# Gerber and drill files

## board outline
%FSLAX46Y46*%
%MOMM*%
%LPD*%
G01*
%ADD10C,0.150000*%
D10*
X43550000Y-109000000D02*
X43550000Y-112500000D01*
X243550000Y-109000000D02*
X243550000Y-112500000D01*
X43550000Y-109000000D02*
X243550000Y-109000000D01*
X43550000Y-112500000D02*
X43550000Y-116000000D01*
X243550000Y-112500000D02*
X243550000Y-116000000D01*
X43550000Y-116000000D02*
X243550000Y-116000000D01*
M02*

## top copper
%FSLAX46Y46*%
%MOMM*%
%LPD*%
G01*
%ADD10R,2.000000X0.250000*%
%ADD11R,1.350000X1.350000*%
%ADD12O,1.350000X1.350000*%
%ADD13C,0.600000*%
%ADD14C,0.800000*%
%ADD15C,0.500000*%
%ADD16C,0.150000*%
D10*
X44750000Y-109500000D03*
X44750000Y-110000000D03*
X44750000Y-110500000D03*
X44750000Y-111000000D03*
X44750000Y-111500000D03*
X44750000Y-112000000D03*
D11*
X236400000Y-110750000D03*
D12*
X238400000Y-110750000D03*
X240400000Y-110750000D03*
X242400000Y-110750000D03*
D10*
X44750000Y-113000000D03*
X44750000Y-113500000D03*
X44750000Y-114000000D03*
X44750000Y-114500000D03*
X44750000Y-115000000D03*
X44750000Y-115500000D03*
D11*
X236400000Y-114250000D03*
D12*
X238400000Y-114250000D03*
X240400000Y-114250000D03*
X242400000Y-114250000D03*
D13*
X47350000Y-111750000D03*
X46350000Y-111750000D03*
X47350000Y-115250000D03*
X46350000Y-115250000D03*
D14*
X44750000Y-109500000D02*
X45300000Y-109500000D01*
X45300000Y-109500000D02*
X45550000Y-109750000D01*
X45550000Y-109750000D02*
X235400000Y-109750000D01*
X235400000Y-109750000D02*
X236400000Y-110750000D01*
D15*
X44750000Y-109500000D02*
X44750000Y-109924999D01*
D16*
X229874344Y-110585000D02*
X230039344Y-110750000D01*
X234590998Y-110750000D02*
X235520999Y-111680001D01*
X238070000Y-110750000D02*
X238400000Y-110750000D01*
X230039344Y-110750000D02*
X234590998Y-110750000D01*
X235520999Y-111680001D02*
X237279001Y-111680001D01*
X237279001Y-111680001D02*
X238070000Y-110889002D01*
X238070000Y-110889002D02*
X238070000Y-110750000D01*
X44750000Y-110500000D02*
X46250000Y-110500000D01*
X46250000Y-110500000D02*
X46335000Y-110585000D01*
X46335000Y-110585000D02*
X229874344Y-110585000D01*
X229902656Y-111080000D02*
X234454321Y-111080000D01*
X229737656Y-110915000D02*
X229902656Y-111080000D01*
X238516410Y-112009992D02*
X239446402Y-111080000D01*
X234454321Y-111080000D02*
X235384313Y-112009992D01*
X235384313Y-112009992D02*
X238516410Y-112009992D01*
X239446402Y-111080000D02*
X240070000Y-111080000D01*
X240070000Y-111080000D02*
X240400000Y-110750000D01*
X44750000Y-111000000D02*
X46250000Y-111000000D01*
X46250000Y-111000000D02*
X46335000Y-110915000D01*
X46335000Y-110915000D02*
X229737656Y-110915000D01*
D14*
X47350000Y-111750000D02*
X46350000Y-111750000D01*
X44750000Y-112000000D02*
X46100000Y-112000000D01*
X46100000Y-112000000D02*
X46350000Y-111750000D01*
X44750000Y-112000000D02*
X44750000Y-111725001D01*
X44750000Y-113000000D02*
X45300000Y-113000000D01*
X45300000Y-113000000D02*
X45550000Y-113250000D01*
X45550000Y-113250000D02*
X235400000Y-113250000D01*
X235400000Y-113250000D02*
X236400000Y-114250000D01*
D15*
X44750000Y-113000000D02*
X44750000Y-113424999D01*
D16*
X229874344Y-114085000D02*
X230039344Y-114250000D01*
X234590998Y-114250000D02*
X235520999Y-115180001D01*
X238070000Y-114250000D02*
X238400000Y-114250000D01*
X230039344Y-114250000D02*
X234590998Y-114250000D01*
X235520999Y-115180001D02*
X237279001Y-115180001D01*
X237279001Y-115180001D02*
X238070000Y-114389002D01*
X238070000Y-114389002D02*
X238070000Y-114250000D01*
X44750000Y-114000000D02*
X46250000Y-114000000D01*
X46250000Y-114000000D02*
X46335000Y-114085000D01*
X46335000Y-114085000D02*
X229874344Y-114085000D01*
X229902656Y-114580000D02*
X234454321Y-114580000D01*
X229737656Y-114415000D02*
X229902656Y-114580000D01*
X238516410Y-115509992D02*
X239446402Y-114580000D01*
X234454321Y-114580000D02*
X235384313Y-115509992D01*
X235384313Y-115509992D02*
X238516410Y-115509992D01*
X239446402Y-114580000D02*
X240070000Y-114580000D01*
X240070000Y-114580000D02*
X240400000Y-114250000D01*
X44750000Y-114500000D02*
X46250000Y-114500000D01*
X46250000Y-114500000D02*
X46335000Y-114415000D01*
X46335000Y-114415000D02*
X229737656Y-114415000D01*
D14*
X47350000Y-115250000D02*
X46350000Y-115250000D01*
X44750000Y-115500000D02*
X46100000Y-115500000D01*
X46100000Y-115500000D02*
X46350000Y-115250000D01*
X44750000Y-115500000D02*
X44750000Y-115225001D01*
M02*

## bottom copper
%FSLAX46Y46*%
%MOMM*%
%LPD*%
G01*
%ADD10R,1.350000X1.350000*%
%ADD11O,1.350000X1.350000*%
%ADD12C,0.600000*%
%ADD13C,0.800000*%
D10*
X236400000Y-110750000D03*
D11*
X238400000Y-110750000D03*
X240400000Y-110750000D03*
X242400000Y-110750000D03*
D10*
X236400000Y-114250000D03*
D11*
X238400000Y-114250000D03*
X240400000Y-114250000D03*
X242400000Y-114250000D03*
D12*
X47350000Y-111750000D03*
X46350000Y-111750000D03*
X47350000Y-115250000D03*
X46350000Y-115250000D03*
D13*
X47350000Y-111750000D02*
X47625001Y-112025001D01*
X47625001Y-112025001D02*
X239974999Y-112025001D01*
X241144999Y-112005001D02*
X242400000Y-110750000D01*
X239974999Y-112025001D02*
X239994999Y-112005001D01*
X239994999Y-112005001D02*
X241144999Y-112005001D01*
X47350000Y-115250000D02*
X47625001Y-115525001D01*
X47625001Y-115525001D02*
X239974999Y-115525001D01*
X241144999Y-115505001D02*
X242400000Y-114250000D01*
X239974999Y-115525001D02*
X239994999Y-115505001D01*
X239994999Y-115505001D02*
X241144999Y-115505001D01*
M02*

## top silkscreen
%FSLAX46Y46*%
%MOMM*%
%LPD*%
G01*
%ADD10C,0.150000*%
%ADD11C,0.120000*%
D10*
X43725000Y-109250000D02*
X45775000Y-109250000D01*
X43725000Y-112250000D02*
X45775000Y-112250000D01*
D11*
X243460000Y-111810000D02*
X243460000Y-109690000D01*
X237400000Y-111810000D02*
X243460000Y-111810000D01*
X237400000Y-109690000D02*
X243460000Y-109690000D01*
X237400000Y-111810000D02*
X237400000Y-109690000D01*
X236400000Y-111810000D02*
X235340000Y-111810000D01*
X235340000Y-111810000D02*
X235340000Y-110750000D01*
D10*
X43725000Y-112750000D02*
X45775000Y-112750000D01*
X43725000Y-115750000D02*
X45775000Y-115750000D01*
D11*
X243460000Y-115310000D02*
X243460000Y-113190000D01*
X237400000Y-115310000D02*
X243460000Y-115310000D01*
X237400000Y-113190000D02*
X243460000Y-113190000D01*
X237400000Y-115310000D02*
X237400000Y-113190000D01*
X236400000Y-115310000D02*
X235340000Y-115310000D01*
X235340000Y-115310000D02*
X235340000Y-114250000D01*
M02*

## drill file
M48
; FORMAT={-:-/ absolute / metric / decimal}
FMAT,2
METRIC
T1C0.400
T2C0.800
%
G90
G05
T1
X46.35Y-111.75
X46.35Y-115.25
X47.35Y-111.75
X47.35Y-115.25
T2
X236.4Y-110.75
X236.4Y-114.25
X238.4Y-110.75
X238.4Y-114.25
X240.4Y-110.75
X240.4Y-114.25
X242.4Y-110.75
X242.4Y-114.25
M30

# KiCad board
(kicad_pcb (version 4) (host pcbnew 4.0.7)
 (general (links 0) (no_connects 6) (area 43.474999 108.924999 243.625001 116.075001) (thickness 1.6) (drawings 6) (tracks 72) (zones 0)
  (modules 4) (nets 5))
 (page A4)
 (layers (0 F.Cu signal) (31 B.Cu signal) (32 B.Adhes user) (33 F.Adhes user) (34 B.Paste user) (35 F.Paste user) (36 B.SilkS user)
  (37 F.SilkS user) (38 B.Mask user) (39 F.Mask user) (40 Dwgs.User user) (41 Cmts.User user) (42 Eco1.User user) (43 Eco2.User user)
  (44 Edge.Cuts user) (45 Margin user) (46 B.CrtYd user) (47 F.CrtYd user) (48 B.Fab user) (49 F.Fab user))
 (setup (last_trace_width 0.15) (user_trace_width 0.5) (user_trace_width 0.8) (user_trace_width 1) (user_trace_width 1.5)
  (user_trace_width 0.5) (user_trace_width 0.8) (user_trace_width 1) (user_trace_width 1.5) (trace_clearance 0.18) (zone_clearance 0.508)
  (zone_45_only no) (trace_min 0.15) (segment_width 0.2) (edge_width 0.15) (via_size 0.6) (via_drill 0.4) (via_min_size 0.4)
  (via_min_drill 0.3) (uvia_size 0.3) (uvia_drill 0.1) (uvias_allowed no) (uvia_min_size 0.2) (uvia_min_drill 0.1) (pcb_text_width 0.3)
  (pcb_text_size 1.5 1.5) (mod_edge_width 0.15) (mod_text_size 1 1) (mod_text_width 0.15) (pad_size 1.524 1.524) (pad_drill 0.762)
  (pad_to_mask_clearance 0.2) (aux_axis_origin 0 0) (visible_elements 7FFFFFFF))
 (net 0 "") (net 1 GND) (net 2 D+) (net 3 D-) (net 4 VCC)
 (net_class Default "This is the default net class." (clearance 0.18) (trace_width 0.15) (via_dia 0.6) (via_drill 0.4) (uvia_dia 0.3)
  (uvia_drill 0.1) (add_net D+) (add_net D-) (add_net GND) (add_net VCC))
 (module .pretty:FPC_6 (layer F.Cu) (at 44.75 110.75 270)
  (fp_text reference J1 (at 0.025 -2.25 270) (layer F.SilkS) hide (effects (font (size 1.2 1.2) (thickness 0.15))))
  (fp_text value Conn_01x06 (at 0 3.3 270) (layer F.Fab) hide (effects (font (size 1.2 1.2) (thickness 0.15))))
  (fp_line (start -1.5 1.025) (end -1.5 -1.025) (layer F.SilkS) (width 0.15))
  (fp_line (start 1.5 1.025) (end 1.5 -1.025) (layer F.SilkS) (width 0.15))
  (pad 1 smd rect (at -1.25 0 270) (size 0.25 2) (layers F.Cu F.Paste F.Mask) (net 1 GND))
  (pad 2 smd rect (at -0.75 0 270) (size 0.25 2) (layers F.Cu F.Paste F.Mask) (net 1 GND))
  (pad 3 smd rect (at -0.25 0 270) (size 0.25 2) (layers F.Cu F.Paste F.Mask) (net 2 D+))
  (pad 4 smd rect (at 0.25 0 270) (size 0.25 2) (layers F.Cu F.Paste F.Mask) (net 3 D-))
  (pad 5 smd rect (at 0.75 0 270) (size 0.25 2) (layers F.Cu F.Paste F.Mask) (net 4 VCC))
  (pad 6 smd rect (at 1.25 0 270) (size 0.25 2) (layers F.Cu F.Paste F.Mask) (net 4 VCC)))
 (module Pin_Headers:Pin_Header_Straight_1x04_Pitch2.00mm (layer F.Cu) (at 236.4 110.75 90)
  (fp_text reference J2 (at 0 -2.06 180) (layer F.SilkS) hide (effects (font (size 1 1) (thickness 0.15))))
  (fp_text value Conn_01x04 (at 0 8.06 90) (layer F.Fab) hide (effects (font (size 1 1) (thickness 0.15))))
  (fp_line (start -1.06 7.06) (end 1.06 7.06) (layer F.SilkS) (width 0.12))
  (fp_line (start -1.06 1) (end -1.06 7.06) (layer F.SilkS) (width 0.12))
  (fp_line (start 1.06 1) (end 1.06 7.06) (layer F.SilkS) (width 0.12))
  (fp_line (start -1.06 1) (end 1.06 1) (layer F.SilkS) (width 0.12))
  (fp_line (start -1.06 0) (end -1.06 -1.06) (layer F.SilkS) (width 0.12))
  (fp_line (start -1.06 -1.06) (end 0 -1.06) (layer F.SilkS) (width 0.12))
  (pad 1 thru_hole rect (at 0 0 90) (size 1.35 1.35) (drill 0.8) (layers *.Cu *.Mask) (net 1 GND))
  (pad 2 thru_hole oval (at 0 2 90) (size 1.35 1.35) (drill 0.8) (layers *.Cu *.Mask) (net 2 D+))
  (pad 3 thru_hole oval (at 0 4 90) (size 1.35 1.35) (drill 0.8) (layers *.Cu *.Mask) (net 3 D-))
  (pad 4 thru_hole oval (at 0 6 90) (size 1.35 1.35) (drill 0.8) (layers *.Cu *.Mask) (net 4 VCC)))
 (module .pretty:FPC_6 (layer F.Cu) (at 44.75 114.25 270)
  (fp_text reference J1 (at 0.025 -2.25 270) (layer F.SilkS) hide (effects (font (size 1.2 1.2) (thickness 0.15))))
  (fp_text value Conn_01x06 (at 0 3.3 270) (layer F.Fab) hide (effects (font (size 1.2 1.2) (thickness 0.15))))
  (fp_line (start -1.5 1.025) (end -1.5 -1.025) (layer F.SilkS) (width 0.15))
  (fp_line (start 1.5 1.025) (end 1.5 -1.025) (layer F.SilkS) (width 0.15))
  (pad 1 smd rect (at -1.25 0 270) (size 0.25 2) (layers F.Cu F.Paste F.Mask) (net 1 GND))
  (pad 2 smd rect (at -0.75 0 270) (size 0.25 2) (layers F.Cu F.Paste F.Mask) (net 1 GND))
  (pad 3 smd rect (at -0.25 0 270) (size 0.25 2) (layers F.Cu F.Paste F.Mask) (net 2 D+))
  (pad 4 smd rect (at 0.25 0 270) (size 0.25 2) (layers F.Cu F.Paste F.Mask) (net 3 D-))
  (pad 5 smd rect (at 0.75 0 270) (size 0.25 2) (layers F.Cu F.Paste F.Mask) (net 4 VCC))
  (pad 6 smd rect (at 1.25 0 270) (size 0.25 2) (layers F.Cu F.Paste F.Mask) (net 4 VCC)))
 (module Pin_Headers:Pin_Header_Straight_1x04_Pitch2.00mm (layer F.Cu) (at 236.4 114.25 90)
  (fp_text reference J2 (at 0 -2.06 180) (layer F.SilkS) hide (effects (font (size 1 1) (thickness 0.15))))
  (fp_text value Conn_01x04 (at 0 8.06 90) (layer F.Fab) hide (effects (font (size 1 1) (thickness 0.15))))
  (fp_line (start -1.06 7.06) (end 1.06 7.06) (layer F.SilkS) (width 0.12))
  (fp_line (start -1.06 1) (end -1.06 7.06) (layer F.SilkS) (width 0.12))
  (fp_line (start 1.06 1) (end 1.06 7.06) (layer F.SilkS) (width 0.12))
  (fp_line (start -1.06 1) (end 1.06 1) (layer F.SilkS) (width 0.12))
  (fp_line (start -1.06 0) (end -1.06 -1.06) (layer F.SilkS) (width 0.12))
  (fp_line (start -1.06 -1.06) (end 0 -1.06) (layer F.SilkS) (width 0.12))
  (pad 1 thru_hole rect (at 0 0 90) (size 1.35 1.35) (drill 0.8) (layers *.Cu *.Mask) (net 1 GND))
  (pad 2 thru_hole oval (at 0 2 90) (size 1.35 1.35) (drill 0.8) (layers *.Cu *.Mask) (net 2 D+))
  (pad 3 thru_hole oval (at 0 4 90) (size 1.35 1.35) (drill 0.8) (layers *.Cu *.Mask) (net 3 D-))
  (pad 4 thru_hole oval (at 0 6 90) (size 1.35 1.35) (drill 0.8) (layers *.Cu *.Mask) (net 4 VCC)))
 (gr_line (start 43.55 109) (end 43.55 112.5) (layer Edge.Cuts) (width 0.15))
 (gr_line (start 243.55 109) (end 243.55 112.5) (layer Edge.Cuts) (width 0.15))
 (gr_line (start 43.55 109) (end 243.55 109) (layer Edge.Cuts) (width 0.15))
 (gr_line (start 43.55 112.5) (end 43.55 116) (layer Edge.Cuts) (width 0.15))
 (gr_line (start 243.55 112.5) (end 243.55 116) (layer Edge.Cuts) (width 0.15))
 (gr_line (start 43.55 116) (end 243.55 116) (layer Edge.Cuts) (width 0.15))
 (segment (start 44.75 109.5) (end 45.3 109.5) (width 0.8) (layer F.Cu) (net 1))
 (segment (start 45.3 109.5) (end 45.55 109.75) (width 0.8) (layer F.Cu) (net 1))
 (segment (start 45.55 109.75) (end 235.4 109.75) (width 0.8) (layer F.Cu) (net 1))
 (segment (start 235.4 109.75) (end 236.4 110.75) (width 0.8) (layer F.Cu) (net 1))
 (segment (start 44.75 109.5) (end 44.75 109.924999) (width 0.5) (layer F.Cu) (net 1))
 (segment (start 229.874344 110.585) (end 230.039344 110.75) (width 0.15) (layer F.Cu) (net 2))
 (segment (start 234.590998 110.75) (end 235.520999 111.680001) (width 0.15) (layer F.Cu) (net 2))
 (segment (start 238.07 110.75) (end 238.4 110.75) (width 0.15) (layer F.Cu) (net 2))
 (segment (start 230.039344 110.75) (end 234.590998 110.75) (width 0.15) (layer F.Cu) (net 2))
 (segment (start 235.520999 111.680001) (end 237.279001 111.680001) (width 0.15) (layer F.Cu) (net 2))
 (segment (start 237.279001 111.680001) (end 238.07 110.889002) (width 0.15) (layer F.Cu) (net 2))
 (segment (start 238.07 110.889002) (end 238.07 110.75) (width 0.15) (layer F.Cu) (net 2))
 (segment (start 44.75 110.5) (end 46.25 110.5) (width 0.15) (layer F.Cu) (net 2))
 (segment (start 46.25 110.5) (end 46.335 110.585) (width 0.15) (layer F.Cu) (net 2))
 (segment (start 46.335 110.585) (end 229.874344 110.585) (width 0.15) (layer F.Cu) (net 2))
 (segment (start 229.902656 111.08) (end 234.454321 111.08) (width 0.15) (layer F.Cu) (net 3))
 (segment (start 229.737656 110.915) (end 229.902656 111.08) (width 0.15) (layer F.Cu) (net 3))
 (segment (start 238.51641 112.009992) (end 239.446402 111.08) (width 0.15) (layer F.Cu) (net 3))
 (segment (start 234.454321 111.08) (end 235.384313 112.009992) (width 0.15) (layer F.Cu) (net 3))
 (segment (start 235.384313 112.009992) (end 238.51641 112.009992) (width 0.15) (layer F.Cu) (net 3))
 (segment (start 239.446402 111.08) (end 240.07 111.08) (width 0.15) (layer F.Cu) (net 3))
 (segment (start 240.07 111.08) (end 240.4 110.75) (width 0.15) (layer F.Cu) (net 3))
 (segment (start 44.75 111) (end 46.25 111) (width 0.15) (layer F.Cu) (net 3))
 (segment (start 46.25 111) (end 46.335 110.915) (width 0.15) (layer F.Cu) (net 3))
 (segment (start 46.335 110.915) (end 229.737656 110.915) (width 0.15) (layer F.Cu) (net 3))
 (segment (start 47.35 111.75) (end 47.625001 112.025001) (width 0.8) (layer B.Cu) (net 4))
 (segment (start 47.625001 112.025001) (end 239.974999 112.025001) (width 0.8) (layer B.Cu) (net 4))
 (segment (start 241.144999 112.005001) (end 242.4 110.75) (width 0.8) (layer B.Cu) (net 4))
 (segment (start 239.974999 112.025001) (end 239.994999 112.005001) (width 0.8) (layer B.Cu) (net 4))
 (segment (start 239.994999 112.005001) (end 241.144999 112.005001) (width 0.8) (layer B.Cu) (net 4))
 (segment (start 47.35 111.75) (end 46.35 111.75) (width 0.8) (layer F.Cu) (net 4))
 (via (at 47.35 111.75) (size 0.6) (drill 0.4) (layers F.Cu B.Cu) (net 4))
 (segment (start 44.75 112) (end 46.1 112) (width 0.8) (layer F.Cu) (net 4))
 (segment (start 46.1 112) (end 46.35 111.75) (width 0.8) (layer F.Cu) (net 4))
 (via (at 46.35 111.75) (size 0.6) (drill 0.4) (layers F.Cu B.Cu) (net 4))
 (segment (start 44.75 112) (end 44.75 111.725001) (width 0.8) (layer F.Cu) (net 4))
 (segment (start 44.75 113) (end 45.3 113) (width 0.8) (layer F.Cu) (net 1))
 (segment (start 45.3 113) (end 45.55 113.25) (width 0.8) (layer F.Cu) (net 1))
 (segment (start 45.55 113.25) (end 235.4 113.25) (width 0.8) (layer F.Cu) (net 1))
 (segment (start 235.4 113.25) (end 236.4 114.25) (width 0.8) (layer F.Cu) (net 1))
 (segment (start 44.75 113) (end 44.75 113.424999) (width 0.5) (layer F.Cu) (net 1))
 (segment (start 229.874344 114.085) (end 230.039344 114.25) (width 0.15) (layer F.Cu) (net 2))
 (segment (start 234.590998 114.25) (end 235.520999 115.180001) (width 0.15) (layer F.Cu) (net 2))
 (segment (start 238.07 114.25) (end 238.4 114.25) (width 0.15) (layer F.Cu) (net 2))
 (segment (start 230.039344 114.25) (end 234.590998 114.25) (width 0.15) (layer F.Cu) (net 2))
 (segment (start 235.520999 115.180001) (end 237.279001 115.180001) (width 0.15) (layer F.Cu) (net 2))
 (segment (start 237.279001 115.180001) (end 238.07 114.389002) (width 0.15) (layer F.Cu) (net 2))
 (segment (start 238.07 114.389002) (end 238.07 114.25) (width 0.15) (layer F.Cu) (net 2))
 (segment (start 44.75 114) (end 46.25 114) (width 0.15) (layer F.Cu) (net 2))
 (segment (start 46.25 114) (end 46.335 114.085) (width 0.15) (layer F.Cu) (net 2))
 (segment (start 46.335 114.085) (end 229.874344 114.085) (width 0.15) (layer F.Cu) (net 2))
 (segment (start 229.902656 114.58) (end 234.454321 114.58) (width 0.15) (layer F.Cu) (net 3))
 (segment (start 229.737656 114.415) (end 229.902656 114.58) (width 0.15) (layer F.Cu) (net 3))
 (segment (start 238.51641 115.509992) (end 239.446402 114.58) (width 0.15) (layer F.Cu) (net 3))
 (segment (start 234.454321 114.58) (end 235.384313 115.509992) (width 0.15) (layer F.Cu) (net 3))
 (segment (start 235.384313 115.509992) (end 238.51641 115.509992) (width 0.15) (layer F.Cu) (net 3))
 (segment (start 239.446402 114.58) (end 240.07 114.58) (width 0.15) (layer F.Cu) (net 3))
 (segment (start 240.07 114.58) (end 240.4 114.25) (width 0.15) (layer F.Cu) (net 3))
 (segment (start 44.75 114.5) (end 46.25 114.5) (width 0.15) (layer F.Cu) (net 3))
 (segment (start 46.25 114.5) (end 46.335 114.415) (width 0.15) (layer F.Cu) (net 3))
 (segment (start 46.335 114.415) (end 229.737656 114.415) (width 0.15) (layer F.Cu) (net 3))
 (segment (start 47.35 115.25) (end 47.625001 115.525001) (width 0.8) (layer B.Cu) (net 4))
 (segment (start 47.625001 115.525001) (end 239.974999 115.525001) (width 0.8) (layer B.Cu) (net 4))
 (segment (start 241.144999 115.505001) (end 242.4 114.25) (width 0.8) (layer B.Cu) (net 4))
 (segment (start 239.974999 115.525001) (end 239.994999 115.505001) (width 0.8) (layer B.Cu) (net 4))
 (segment (start 239.994999 115.505001) (end 241.144999 115.505001) (width 0.8) (layer B.Cu) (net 4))
 (segment (start 47.35 115.25) (end 46.35 115.25) (width 0.8) (layer F.Cu) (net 4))
 (via (at 47.35 115.25) (size 0.6) (drill 0.4) (layers F.Cu B.Cu) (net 4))
 (segment (start 44.75 115.5) (end 46.1 115.5) (width 0.8) (layer F.Cu) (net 4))
 (segment (start 46.1 115.5) (end 46.35 115.25) (width 0.8) (layer F.Cu) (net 4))
 (via (at 46.35 115.25) (size 0.6) (drill 0.4) (layers F.Cu B.Cu) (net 4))
 (segment (start 44.75 115.5) (end 44.75 115.225001) (width 0.8) (layer F.Cu) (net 4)))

